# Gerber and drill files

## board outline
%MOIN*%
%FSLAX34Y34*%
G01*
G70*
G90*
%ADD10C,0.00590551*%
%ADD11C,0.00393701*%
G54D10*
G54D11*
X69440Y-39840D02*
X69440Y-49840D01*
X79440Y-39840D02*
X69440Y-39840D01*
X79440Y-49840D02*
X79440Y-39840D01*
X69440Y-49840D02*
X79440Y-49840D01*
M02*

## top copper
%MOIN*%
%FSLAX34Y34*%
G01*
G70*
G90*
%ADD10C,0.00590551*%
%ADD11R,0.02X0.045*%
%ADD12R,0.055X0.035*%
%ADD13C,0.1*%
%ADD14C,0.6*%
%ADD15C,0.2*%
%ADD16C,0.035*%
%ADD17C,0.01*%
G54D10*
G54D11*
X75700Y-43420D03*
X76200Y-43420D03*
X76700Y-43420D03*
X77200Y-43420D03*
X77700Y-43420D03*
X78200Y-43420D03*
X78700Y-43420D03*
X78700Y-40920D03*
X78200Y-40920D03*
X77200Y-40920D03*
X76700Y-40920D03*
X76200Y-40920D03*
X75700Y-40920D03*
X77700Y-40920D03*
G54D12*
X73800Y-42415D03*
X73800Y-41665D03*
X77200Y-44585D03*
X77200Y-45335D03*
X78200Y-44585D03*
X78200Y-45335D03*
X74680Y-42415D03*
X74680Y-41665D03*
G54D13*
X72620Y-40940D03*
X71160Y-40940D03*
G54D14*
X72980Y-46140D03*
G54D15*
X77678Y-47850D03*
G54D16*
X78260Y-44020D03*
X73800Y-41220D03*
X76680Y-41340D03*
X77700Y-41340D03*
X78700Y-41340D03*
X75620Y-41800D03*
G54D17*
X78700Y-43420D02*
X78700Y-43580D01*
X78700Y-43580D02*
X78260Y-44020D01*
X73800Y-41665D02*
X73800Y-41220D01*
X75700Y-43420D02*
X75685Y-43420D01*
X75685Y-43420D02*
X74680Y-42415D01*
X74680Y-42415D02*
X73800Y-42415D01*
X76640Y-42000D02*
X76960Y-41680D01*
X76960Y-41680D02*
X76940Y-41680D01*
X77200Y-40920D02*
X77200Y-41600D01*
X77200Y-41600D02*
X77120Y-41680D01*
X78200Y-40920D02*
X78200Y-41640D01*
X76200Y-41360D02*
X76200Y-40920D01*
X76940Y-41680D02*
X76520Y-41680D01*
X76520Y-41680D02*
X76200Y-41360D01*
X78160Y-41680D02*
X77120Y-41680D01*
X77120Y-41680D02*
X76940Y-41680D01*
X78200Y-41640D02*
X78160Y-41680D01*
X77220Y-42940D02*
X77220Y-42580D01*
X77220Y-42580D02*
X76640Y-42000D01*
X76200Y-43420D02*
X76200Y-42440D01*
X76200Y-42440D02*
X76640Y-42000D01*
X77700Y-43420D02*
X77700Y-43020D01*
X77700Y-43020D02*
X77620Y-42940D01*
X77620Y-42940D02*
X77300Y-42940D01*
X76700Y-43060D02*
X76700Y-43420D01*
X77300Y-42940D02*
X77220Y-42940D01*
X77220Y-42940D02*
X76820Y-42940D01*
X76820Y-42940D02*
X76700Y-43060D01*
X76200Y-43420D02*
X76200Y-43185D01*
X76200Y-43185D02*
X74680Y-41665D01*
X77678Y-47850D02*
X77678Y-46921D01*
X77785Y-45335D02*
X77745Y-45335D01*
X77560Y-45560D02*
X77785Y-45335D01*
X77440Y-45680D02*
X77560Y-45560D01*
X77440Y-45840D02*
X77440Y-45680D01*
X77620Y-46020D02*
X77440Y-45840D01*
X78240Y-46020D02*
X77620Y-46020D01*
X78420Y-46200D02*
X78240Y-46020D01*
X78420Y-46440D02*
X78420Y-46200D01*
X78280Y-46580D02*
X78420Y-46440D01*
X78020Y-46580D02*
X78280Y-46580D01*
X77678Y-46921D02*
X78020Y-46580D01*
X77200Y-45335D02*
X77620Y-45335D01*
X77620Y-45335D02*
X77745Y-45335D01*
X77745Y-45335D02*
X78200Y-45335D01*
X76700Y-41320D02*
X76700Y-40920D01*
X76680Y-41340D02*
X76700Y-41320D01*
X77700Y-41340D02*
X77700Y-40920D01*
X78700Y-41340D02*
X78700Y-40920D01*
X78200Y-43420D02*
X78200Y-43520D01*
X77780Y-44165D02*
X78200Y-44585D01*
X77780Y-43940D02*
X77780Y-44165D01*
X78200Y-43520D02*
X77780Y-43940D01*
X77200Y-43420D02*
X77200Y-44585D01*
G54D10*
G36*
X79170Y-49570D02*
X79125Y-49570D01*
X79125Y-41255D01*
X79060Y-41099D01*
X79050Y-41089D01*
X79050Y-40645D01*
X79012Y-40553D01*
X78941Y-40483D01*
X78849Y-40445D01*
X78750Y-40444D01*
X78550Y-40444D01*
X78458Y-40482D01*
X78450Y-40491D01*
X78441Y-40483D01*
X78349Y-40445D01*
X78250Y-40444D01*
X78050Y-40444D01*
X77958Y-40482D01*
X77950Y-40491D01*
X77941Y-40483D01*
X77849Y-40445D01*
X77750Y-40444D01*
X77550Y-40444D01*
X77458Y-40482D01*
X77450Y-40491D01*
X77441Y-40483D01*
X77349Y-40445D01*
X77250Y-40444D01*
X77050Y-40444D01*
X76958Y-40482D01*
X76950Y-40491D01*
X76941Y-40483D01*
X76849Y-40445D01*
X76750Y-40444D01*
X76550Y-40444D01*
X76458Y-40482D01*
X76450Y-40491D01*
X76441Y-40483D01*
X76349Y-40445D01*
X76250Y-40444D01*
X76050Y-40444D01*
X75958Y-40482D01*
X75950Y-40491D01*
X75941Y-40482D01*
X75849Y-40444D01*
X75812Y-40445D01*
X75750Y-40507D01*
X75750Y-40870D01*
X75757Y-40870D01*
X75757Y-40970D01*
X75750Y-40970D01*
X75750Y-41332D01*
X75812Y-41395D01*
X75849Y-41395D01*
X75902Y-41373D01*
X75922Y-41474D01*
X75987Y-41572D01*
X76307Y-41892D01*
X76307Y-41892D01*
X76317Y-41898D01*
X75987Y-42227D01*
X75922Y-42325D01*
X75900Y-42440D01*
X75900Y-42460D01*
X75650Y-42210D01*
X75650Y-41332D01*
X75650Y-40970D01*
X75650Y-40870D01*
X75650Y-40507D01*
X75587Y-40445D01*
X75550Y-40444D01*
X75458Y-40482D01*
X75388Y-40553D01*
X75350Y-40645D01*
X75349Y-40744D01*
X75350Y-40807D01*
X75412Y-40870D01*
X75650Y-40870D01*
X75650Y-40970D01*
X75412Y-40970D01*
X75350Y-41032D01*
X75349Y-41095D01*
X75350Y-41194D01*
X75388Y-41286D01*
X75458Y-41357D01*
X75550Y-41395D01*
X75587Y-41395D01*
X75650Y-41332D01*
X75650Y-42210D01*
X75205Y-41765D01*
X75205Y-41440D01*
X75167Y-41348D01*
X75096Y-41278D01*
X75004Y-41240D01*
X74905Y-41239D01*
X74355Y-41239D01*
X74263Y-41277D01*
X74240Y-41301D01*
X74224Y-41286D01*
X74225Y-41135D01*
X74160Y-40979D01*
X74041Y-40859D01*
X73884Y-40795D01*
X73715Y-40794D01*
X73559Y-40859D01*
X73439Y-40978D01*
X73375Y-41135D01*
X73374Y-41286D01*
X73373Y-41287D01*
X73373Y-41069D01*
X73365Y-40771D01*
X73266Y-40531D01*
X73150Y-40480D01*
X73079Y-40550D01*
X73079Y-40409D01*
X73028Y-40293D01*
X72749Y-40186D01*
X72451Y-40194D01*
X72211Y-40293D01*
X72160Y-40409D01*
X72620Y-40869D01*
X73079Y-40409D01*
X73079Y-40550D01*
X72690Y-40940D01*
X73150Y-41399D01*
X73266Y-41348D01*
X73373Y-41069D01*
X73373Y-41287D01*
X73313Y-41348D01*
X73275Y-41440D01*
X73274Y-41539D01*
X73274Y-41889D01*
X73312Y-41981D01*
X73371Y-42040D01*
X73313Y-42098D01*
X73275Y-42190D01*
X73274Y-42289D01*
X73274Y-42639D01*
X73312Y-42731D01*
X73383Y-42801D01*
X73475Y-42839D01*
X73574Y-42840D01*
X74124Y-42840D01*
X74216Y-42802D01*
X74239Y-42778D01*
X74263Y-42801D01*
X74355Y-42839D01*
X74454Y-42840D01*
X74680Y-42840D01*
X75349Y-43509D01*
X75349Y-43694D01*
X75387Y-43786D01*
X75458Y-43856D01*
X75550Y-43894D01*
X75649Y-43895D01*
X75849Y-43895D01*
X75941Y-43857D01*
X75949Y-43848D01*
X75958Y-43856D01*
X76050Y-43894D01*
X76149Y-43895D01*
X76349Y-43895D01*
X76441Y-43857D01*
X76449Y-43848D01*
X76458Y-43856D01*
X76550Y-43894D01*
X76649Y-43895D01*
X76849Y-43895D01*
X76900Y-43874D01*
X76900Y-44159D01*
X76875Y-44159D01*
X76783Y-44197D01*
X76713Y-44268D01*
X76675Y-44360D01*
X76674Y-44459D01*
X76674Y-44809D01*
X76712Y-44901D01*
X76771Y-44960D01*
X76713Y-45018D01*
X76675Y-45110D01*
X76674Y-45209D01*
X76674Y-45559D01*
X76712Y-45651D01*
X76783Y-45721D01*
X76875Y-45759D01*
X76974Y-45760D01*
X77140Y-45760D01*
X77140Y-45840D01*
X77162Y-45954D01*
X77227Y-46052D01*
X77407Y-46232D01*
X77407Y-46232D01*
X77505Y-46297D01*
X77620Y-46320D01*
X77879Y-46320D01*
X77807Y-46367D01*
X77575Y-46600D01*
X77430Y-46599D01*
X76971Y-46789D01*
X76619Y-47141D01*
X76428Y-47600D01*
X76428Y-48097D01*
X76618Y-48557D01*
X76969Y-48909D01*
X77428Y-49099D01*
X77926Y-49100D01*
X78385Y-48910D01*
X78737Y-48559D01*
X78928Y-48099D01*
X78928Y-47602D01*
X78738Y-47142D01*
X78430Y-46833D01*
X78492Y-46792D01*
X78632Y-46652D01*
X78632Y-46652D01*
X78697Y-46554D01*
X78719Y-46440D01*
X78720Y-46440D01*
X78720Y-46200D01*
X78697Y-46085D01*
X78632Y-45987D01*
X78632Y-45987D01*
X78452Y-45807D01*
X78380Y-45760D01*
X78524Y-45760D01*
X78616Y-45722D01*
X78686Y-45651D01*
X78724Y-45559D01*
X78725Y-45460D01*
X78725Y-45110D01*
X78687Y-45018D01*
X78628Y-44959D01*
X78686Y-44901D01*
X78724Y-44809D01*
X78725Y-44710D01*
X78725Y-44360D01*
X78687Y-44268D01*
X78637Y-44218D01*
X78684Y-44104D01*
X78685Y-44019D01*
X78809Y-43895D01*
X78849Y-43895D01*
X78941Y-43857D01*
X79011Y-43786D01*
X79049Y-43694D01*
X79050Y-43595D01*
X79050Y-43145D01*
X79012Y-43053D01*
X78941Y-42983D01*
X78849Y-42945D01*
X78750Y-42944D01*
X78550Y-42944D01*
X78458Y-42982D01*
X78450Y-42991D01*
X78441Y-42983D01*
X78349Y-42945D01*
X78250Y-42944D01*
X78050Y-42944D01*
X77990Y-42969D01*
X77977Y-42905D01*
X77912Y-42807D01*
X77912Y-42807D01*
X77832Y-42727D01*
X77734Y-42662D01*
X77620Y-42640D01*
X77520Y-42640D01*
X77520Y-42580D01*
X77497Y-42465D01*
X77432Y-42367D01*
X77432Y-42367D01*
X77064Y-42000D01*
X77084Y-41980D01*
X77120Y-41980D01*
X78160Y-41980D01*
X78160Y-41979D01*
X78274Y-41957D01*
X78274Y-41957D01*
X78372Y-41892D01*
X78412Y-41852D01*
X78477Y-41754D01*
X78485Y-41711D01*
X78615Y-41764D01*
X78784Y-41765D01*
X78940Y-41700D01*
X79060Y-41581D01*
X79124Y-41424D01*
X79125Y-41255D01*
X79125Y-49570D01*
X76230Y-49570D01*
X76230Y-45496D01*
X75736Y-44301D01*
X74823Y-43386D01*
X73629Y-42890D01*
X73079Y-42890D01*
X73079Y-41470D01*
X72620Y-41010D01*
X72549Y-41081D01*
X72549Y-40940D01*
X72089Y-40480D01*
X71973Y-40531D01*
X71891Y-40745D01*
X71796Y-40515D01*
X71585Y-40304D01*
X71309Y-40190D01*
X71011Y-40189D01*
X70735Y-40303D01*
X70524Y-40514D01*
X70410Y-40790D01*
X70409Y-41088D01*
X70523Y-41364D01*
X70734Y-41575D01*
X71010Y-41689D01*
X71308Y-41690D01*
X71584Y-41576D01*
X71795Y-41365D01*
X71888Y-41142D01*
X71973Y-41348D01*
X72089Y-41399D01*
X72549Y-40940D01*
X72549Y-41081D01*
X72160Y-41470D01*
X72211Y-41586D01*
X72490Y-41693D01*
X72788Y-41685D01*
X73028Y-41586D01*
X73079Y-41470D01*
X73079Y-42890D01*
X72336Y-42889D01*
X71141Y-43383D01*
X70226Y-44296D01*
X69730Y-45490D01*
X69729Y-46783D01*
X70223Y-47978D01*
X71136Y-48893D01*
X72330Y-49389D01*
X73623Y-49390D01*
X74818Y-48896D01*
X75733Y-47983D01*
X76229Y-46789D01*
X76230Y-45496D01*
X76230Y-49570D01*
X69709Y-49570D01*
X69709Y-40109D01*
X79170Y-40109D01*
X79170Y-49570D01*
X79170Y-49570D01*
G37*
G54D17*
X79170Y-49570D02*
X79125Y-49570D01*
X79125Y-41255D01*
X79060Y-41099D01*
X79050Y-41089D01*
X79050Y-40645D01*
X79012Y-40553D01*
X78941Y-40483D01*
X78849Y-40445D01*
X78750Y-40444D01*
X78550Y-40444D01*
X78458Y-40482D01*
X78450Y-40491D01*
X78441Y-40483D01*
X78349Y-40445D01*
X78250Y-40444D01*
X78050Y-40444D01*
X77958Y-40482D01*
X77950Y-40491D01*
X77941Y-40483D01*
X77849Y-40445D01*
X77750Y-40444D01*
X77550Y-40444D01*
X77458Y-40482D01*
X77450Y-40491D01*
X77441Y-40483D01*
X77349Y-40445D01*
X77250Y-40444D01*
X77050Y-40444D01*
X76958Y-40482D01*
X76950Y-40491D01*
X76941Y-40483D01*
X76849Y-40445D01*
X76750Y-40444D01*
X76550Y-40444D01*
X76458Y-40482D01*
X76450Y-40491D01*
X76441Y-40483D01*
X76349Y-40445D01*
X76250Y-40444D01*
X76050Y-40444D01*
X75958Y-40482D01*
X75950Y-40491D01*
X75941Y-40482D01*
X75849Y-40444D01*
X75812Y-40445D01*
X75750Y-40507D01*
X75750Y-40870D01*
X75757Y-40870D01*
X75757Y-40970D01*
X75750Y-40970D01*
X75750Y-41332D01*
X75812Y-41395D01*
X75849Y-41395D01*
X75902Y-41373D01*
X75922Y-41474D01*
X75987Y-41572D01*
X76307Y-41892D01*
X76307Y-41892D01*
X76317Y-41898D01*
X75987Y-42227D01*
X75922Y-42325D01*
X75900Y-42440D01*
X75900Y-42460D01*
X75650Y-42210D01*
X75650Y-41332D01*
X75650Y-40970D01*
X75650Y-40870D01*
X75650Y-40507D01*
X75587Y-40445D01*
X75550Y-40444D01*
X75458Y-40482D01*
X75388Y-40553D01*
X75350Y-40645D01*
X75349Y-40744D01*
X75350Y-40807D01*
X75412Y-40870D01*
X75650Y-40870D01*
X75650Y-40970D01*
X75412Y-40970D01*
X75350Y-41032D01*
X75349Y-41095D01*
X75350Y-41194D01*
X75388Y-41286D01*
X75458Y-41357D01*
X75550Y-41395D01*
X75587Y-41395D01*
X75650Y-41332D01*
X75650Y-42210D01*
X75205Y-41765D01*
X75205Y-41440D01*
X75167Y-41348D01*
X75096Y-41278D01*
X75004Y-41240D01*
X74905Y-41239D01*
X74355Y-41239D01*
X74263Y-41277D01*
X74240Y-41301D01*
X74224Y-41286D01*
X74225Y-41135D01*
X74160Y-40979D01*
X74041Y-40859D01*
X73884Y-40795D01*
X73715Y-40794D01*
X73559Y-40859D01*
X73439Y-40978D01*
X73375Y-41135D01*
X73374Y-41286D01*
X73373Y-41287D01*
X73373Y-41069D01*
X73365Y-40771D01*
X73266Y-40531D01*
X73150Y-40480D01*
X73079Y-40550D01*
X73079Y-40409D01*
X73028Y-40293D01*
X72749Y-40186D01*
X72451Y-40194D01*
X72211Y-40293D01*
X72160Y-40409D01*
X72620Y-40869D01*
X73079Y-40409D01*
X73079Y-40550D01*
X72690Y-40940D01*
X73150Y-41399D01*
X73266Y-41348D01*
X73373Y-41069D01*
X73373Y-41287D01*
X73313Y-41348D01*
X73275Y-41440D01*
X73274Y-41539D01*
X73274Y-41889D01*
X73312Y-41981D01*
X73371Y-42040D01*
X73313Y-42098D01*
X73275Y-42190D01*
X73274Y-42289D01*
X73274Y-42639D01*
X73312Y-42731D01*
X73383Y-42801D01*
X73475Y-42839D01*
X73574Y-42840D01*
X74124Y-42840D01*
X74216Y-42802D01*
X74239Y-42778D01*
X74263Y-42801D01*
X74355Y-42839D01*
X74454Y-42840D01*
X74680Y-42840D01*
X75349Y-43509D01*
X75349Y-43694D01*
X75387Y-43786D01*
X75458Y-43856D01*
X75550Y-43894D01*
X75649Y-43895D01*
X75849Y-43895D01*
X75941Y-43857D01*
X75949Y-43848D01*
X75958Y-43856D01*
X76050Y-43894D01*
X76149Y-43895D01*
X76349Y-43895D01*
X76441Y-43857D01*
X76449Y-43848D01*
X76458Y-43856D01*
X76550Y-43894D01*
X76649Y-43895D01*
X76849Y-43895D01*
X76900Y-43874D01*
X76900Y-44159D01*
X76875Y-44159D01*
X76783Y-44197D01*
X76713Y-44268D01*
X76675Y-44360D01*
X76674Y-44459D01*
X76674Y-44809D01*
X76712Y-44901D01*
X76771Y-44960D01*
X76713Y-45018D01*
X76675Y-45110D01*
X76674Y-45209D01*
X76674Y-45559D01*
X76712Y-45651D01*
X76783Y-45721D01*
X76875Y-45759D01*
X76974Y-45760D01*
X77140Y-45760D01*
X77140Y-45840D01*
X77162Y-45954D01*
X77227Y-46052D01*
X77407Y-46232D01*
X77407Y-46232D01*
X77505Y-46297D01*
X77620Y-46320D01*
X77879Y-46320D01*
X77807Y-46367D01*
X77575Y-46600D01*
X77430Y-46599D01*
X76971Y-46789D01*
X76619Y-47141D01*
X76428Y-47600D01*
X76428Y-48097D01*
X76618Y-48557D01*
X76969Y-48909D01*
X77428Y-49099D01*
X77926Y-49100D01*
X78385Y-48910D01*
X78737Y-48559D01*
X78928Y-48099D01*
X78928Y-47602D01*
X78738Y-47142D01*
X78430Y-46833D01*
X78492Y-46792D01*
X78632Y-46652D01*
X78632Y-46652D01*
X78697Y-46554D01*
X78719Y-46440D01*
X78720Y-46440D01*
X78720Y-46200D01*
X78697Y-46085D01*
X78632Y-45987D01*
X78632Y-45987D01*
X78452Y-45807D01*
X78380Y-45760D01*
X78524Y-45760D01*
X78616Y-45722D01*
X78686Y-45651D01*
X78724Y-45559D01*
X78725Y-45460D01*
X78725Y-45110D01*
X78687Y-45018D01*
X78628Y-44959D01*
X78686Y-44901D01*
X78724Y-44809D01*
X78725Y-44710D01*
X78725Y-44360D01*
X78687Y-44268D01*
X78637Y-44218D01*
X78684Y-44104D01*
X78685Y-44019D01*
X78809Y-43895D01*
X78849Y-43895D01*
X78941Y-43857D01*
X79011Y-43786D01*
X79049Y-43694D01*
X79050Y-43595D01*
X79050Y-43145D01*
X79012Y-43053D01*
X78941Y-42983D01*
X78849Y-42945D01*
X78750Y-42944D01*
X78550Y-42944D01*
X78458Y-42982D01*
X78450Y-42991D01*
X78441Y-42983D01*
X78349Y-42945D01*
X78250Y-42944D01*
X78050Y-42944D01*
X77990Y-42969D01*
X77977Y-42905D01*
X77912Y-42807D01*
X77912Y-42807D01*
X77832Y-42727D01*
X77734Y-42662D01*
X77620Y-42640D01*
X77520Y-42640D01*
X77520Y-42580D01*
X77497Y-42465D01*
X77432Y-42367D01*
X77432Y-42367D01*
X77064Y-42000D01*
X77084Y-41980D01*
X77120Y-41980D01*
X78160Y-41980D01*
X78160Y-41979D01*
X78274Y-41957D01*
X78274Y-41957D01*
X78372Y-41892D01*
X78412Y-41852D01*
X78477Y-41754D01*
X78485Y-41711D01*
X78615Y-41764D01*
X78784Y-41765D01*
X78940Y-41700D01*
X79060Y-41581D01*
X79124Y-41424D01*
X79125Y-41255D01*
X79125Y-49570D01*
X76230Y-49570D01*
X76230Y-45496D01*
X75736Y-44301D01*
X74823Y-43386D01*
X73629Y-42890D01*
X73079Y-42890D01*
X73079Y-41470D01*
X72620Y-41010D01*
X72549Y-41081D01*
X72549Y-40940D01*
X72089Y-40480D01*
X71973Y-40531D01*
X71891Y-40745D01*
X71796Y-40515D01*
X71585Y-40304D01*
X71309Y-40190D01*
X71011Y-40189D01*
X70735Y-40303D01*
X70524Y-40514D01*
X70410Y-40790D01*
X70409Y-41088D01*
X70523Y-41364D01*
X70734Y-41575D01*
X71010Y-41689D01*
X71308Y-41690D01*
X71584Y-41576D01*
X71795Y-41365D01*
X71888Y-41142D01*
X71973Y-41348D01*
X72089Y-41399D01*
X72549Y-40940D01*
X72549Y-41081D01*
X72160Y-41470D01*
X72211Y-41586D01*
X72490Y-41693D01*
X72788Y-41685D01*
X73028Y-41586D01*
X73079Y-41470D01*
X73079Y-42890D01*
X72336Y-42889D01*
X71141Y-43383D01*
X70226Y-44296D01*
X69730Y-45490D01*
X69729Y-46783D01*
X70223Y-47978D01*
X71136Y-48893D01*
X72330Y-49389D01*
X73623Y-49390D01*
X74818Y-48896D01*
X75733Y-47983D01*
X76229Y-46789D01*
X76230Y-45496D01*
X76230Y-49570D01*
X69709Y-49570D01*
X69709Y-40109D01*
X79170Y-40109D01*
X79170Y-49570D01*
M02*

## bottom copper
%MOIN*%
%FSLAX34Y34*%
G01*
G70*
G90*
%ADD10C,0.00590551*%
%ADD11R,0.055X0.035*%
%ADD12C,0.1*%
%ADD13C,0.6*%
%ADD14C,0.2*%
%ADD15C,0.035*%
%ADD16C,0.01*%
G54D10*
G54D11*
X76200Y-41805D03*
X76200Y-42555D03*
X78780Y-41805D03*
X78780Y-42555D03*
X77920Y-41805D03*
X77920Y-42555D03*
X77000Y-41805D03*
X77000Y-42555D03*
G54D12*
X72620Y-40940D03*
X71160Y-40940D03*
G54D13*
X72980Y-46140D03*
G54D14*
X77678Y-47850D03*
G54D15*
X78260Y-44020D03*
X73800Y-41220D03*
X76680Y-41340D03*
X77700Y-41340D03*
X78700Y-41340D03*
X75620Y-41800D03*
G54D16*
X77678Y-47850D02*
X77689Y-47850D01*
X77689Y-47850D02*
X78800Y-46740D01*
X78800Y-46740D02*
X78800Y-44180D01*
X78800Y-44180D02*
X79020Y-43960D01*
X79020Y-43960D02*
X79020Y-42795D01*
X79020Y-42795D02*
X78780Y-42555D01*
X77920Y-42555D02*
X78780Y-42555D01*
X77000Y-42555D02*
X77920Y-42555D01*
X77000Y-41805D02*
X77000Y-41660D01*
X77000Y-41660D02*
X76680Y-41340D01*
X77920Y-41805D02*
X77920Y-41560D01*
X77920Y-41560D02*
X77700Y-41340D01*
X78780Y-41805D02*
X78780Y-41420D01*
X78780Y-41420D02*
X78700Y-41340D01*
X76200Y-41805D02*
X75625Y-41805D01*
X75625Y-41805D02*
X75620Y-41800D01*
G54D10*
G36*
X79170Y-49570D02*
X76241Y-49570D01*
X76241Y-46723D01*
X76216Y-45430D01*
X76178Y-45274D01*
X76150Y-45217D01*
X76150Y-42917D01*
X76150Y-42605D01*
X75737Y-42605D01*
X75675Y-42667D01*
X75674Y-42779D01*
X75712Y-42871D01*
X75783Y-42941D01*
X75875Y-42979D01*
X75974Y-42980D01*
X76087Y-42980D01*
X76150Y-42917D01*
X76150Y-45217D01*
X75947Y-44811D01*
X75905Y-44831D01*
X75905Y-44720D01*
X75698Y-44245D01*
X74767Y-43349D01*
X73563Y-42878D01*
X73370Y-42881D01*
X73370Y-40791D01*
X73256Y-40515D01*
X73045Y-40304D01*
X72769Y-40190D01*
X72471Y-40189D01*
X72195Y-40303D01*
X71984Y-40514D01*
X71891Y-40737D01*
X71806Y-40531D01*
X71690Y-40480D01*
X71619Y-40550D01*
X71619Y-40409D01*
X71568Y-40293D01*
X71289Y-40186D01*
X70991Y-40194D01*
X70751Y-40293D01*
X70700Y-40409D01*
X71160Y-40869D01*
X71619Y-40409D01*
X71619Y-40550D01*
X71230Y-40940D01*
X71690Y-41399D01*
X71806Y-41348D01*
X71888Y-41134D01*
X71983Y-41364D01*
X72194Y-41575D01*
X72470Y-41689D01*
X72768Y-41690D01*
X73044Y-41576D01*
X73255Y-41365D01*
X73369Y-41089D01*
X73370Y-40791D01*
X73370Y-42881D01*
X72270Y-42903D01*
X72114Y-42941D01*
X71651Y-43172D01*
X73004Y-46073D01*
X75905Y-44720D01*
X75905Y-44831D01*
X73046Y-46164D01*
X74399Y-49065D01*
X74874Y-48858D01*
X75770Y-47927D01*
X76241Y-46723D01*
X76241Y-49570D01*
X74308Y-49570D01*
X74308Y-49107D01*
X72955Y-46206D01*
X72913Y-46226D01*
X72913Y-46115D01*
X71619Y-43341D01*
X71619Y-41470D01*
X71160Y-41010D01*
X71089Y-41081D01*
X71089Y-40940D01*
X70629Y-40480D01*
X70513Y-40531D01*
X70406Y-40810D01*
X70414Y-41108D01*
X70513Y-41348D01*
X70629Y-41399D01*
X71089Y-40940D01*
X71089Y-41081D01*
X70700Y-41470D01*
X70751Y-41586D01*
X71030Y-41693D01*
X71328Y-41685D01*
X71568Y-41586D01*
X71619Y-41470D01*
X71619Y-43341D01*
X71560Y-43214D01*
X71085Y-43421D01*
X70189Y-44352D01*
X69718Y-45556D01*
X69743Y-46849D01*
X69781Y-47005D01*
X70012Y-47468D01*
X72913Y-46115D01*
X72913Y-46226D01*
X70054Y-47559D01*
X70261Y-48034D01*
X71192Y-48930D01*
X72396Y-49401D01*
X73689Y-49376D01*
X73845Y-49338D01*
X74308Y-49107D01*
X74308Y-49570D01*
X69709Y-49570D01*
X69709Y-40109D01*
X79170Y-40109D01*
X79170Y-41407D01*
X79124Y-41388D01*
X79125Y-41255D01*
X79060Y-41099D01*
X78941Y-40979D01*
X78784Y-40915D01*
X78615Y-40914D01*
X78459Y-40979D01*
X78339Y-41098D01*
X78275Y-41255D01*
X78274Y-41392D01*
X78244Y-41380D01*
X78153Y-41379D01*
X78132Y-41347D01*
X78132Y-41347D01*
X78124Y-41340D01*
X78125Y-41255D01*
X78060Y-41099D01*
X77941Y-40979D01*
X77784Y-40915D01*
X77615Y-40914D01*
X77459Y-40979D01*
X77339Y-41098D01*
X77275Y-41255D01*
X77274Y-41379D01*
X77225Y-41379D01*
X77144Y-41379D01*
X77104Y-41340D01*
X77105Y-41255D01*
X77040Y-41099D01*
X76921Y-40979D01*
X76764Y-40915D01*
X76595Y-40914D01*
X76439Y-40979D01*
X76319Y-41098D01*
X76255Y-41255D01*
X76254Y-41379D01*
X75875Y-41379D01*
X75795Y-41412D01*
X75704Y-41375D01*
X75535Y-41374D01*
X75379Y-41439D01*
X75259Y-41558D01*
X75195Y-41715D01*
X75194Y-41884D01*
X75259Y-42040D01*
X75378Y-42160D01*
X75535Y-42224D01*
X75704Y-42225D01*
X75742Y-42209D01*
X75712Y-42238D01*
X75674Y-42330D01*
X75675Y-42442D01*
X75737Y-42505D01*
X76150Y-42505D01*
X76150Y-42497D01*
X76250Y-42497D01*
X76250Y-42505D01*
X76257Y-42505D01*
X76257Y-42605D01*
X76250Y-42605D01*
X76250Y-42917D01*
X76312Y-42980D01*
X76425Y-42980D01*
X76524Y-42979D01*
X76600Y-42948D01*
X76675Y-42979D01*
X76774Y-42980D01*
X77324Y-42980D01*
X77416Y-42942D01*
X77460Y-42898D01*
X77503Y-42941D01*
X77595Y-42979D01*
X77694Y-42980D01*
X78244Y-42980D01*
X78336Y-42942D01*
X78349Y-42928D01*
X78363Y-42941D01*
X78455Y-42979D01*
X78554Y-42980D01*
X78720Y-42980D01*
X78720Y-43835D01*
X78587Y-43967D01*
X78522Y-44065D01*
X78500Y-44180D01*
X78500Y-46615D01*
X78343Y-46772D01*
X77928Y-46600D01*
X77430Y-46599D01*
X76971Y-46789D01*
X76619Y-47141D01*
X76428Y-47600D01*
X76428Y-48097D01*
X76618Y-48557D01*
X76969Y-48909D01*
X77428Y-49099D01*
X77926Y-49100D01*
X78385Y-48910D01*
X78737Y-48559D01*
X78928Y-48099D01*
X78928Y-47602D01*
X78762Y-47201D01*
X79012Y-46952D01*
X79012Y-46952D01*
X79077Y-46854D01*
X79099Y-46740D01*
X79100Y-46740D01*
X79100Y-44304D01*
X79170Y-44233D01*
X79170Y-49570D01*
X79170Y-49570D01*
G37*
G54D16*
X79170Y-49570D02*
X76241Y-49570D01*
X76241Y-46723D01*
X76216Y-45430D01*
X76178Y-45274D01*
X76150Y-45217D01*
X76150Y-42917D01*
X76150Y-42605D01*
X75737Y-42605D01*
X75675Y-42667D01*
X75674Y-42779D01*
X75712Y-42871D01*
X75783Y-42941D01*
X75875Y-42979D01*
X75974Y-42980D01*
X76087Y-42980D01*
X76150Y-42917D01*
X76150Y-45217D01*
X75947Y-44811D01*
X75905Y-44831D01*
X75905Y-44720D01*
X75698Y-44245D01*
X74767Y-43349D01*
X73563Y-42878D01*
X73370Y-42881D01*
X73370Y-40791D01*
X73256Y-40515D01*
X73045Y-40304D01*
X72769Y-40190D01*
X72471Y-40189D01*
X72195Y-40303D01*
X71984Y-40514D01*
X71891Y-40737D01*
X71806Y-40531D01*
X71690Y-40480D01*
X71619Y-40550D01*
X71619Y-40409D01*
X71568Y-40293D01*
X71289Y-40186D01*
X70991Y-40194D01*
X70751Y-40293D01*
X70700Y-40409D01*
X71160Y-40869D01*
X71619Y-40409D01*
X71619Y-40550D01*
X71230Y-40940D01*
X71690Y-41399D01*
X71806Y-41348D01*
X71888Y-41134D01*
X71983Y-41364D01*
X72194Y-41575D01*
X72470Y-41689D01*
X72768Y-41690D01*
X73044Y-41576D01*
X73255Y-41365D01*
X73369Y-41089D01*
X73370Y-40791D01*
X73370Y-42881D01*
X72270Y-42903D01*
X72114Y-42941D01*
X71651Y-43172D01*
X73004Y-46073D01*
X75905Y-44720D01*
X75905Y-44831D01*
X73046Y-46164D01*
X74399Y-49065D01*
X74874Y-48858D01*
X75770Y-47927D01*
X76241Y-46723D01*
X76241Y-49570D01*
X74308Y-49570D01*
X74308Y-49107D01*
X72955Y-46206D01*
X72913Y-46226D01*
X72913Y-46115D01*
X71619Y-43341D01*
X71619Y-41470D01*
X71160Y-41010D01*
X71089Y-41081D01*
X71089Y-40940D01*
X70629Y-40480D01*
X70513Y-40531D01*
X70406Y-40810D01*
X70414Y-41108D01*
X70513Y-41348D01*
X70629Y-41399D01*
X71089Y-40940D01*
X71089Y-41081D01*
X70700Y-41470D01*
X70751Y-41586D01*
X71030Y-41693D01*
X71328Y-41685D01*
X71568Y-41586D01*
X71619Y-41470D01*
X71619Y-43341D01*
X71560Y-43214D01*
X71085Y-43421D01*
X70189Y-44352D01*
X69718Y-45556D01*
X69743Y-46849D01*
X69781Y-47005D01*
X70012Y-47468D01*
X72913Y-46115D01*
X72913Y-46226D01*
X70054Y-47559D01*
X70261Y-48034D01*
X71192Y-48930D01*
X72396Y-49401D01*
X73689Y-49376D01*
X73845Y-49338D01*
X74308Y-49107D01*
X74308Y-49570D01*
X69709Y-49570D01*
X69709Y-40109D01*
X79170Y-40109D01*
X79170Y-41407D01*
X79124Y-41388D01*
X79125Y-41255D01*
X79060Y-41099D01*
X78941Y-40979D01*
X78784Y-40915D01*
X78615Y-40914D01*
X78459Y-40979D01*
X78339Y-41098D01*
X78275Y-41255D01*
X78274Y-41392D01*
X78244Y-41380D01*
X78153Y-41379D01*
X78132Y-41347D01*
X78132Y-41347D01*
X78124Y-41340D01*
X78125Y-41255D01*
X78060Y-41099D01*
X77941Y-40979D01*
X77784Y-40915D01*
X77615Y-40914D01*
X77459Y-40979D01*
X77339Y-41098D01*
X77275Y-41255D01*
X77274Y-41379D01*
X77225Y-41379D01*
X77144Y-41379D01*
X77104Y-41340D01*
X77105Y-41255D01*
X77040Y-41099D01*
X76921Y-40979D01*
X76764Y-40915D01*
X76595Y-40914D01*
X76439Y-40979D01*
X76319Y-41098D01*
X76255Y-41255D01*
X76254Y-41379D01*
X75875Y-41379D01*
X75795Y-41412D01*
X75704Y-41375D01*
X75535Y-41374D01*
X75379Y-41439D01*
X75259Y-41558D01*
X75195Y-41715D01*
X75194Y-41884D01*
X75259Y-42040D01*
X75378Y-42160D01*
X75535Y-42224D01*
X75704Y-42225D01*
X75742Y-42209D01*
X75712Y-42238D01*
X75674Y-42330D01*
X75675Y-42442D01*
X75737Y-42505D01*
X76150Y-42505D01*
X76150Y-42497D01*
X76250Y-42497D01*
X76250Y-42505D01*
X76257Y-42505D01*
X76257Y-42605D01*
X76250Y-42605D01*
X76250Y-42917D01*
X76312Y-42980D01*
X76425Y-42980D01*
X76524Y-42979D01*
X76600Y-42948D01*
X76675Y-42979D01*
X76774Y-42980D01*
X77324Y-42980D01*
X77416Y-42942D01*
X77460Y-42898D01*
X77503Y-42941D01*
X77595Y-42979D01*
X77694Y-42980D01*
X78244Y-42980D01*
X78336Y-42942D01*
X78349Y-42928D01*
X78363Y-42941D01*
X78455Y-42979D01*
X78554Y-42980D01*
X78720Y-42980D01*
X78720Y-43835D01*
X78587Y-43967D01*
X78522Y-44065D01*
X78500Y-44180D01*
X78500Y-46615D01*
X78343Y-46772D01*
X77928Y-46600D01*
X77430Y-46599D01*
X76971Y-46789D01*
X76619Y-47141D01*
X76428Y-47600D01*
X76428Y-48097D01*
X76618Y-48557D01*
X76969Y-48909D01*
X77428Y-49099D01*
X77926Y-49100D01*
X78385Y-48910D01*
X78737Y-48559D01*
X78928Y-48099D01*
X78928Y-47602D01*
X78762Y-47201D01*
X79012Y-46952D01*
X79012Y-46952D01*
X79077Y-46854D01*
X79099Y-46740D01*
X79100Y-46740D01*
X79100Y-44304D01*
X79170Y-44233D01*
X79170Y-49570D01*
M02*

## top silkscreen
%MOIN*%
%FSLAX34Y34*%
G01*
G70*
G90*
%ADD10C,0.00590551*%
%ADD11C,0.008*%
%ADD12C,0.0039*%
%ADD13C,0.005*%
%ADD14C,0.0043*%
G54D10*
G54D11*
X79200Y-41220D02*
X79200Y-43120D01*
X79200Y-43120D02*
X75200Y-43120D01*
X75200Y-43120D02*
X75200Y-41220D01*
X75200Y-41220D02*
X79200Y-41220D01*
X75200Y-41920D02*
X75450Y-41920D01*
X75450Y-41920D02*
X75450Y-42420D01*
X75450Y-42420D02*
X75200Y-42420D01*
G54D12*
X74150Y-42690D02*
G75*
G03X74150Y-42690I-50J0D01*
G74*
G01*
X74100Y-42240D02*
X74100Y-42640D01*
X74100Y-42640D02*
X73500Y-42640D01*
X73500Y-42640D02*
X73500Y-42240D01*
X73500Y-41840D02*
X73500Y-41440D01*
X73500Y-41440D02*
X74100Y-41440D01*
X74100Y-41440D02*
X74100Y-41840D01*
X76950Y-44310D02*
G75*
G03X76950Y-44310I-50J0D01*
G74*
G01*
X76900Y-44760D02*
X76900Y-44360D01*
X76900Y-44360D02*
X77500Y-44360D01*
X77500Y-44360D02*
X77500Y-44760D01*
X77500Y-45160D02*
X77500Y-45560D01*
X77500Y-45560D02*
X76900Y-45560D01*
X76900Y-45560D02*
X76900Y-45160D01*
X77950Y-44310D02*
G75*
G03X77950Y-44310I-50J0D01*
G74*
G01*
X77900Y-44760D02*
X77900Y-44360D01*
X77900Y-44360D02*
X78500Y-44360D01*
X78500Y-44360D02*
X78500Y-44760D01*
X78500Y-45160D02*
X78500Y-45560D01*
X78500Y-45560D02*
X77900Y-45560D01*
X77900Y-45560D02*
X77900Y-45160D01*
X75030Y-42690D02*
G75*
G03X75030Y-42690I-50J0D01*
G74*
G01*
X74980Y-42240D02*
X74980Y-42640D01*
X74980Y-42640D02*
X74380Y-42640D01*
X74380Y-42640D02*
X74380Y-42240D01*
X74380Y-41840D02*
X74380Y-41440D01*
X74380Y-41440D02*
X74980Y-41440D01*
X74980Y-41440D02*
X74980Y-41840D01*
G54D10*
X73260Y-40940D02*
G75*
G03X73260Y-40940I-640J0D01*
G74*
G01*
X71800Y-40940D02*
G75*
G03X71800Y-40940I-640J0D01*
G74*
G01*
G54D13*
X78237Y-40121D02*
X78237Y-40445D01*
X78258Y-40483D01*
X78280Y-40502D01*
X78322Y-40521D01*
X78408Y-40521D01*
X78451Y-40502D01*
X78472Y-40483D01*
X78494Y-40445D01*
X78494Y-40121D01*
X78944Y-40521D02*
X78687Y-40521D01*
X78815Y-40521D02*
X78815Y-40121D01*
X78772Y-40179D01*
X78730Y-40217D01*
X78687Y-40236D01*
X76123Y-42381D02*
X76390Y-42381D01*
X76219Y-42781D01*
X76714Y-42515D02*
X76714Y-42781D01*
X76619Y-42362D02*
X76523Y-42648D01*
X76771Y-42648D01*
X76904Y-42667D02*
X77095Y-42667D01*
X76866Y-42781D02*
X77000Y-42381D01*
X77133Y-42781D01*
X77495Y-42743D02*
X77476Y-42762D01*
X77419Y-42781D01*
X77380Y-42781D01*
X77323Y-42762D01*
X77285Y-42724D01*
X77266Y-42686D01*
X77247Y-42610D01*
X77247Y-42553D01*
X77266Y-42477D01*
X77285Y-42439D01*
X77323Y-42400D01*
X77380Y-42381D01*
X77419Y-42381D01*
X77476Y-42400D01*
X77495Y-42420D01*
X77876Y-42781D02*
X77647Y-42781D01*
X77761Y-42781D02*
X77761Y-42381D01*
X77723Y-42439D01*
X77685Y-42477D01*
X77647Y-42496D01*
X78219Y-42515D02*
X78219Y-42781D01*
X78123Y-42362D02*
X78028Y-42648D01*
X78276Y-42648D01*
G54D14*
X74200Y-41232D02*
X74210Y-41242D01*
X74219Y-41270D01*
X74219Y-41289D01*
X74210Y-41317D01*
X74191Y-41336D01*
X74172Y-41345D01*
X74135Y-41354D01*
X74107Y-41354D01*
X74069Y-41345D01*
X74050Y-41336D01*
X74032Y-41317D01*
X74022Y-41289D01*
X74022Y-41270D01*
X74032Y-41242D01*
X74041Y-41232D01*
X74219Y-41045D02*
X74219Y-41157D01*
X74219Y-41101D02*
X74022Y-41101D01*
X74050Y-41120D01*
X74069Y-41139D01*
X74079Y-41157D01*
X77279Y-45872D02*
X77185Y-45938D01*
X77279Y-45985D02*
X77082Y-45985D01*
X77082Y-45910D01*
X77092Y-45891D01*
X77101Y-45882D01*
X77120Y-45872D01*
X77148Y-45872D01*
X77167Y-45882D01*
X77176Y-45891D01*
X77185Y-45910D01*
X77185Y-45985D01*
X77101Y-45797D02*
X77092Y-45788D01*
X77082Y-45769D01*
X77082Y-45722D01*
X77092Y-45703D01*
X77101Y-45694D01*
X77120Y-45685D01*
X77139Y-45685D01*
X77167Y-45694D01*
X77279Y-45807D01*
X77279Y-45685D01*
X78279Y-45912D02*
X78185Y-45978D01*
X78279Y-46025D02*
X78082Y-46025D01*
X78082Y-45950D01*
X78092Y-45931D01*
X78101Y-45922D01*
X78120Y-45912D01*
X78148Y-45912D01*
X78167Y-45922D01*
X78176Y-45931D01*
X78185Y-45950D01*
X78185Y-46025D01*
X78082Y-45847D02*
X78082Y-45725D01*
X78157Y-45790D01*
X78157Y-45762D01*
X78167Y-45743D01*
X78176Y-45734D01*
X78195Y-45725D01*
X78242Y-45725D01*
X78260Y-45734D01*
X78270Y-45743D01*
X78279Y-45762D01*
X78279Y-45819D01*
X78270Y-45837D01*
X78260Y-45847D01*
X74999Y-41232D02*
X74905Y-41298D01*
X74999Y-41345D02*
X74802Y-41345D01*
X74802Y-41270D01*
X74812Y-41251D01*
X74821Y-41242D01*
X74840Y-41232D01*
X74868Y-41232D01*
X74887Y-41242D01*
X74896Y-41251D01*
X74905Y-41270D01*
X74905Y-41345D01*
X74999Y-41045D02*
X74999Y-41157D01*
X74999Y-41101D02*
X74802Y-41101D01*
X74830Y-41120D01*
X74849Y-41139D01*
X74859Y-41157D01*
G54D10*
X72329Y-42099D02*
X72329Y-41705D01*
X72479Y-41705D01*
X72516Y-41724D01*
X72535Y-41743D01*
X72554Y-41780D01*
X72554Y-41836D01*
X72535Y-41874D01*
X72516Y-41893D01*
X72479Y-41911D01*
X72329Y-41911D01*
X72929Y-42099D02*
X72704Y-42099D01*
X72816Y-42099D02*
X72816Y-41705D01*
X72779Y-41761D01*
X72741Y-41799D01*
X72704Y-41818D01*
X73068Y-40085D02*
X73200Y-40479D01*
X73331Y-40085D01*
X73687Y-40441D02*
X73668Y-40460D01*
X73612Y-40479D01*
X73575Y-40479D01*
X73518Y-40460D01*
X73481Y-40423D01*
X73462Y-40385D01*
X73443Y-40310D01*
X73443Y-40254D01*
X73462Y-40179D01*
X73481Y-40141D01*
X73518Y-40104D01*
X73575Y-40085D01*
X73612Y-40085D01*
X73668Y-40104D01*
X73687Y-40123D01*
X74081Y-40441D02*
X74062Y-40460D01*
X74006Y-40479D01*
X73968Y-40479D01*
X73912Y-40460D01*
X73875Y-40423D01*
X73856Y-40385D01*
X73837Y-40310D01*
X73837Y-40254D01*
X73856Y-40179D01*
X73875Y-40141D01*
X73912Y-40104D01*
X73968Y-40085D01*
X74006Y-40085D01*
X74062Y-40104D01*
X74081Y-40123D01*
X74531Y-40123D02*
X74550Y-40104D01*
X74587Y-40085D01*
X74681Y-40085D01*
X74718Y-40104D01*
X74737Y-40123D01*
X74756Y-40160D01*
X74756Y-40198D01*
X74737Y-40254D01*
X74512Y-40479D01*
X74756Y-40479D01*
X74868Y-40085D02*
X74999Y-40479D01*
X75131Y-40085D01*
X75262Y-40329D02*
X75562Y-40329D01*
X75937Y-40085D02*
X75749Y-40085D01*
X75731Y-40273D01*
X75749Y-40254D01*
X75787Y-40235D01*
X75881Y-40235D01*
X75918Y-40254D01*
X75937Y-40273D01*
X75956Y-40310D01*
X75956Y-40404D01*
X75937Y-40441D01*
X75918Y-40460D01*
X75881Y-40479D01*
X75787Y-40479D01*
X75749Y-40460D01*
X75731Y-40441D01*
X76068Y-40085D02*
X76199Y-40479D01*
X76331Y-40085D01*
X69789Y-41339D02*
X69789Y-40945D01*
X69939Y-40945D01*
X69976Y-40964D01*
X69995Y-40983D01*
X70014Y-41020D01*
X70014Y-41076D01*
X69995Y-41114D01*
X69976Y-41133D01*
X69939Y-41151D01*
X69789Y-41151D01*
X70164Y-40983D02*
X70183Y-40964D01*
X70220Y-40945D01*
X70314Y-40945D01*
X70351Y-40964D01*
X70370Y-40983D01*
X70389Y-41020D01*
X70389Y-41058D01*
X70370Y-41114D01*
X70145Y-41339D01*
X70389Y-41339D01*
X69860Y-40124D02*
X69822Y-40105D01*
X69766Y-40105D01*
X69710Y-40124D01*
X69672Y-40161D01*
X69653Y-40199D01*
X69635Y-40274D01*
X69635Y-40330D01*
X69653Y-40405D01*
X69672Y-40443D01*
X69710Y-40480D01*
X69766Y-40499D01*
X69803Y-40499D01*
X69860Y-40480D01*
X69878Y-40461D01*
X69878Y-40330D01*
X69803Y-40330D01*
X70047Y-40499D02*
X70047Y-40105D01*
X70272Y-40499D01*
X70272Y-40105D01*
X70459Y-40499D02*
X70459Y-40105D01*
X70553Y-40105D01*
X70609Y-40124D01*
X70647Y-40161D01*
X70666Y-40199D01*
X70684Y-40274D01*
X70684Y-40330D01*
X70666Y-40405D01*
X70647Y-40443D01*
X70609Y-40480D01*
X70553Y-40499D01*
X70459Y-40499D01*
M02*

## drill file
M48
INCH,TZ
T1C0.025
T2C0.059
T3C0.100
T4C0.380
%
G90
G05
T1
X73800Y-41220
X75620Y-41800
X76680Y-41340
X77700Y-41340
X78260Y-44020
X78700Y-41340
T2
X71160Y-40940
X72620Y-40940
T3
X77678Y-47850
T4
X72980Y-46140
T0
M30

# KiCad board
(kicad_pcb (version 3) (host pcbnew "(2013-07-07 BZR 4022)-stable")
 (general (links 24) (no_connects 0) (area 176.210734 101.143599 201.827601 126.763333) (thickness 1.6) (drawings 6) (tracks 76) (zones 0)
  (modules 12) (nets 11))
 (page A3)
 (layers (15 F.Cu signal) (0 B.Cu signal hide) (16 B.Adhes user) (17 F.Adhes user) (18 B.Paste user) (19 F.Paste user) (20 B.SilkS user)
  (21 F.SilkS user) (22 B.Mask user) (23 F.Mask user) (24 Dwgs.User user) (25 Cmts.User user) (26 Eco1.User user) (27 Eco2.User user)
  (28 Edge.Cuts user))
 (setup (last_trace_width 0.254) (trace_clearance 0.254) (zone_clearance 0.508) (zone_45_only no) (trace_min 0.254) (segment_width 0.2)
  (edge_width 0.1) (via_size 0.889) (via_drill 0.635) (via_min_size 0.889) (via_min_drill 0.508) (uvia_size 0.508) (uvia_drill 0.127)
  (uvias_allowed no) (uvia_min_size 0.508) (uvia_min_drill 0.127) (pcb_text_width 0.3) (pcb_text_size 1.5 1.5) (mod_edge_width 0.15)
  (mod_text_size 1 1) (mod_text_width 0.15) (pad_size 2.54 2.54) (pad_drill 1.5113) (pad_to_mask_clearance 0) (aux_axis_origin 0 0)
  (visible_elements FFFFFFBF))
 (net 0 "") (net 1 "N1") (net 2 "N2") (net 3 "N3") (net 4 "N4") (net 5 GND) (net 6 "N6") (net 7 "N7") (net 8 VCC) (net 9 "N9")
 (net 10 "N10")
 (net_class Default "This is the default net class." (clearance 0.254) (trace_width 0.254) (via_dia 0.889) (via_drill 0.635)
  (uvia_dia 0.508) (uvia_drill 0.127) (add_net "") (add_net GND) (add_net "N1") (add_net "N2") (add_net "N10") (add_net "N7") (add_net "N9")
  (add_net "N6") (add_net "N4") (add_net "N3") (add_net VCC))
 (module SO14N (layer F.Cu) (at 196.088 106.9848)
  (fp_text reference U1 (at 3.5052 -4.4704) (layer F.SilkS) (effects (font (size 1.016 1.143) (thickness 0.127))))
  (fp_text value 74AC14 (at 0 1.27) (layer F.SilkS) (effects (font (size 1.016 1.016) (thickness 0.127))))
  (fp_line (start 5.08 -2.286) (end 5.08 2.54) (layer F.SilkS) (width 0.2032))
  (fp_line (start 5.08 2.54) (end -5.08 2.54) (layer F.SilkS) (width 0.2032))
  (fp_line (start -5.08 2.54) (end -5.08 -2.286) (layer F.SilkS) (width 0.2032))
  (fp_line (start -5.08 -2.286) (end 5.08 -2.286) (layer F.SilkS) (width 0.2032))
  (fp_line (start -5.08 -0.508) (end -4.445 -0.508) (layer F.SilkS) (width 0.2032))
  (fp_line (start -4.445 -0.508) (end -4.445 0.762) (layer F.SilkS) (width 0.2032))
  (fp_line (start -4.445 0.762) (end -5.08 0.762) (layer F.SilkS) (width 0.2032))
  (pad 1 smd rect (at -3.81 3.302) (size 0.508 1.143) (layers F.Cu F.Paste F.Mask) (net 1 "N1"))
  (pad 2 smd rect (at -2.54 3.302) (size 0.508 1.143) (layers F.Cu F.Paste F.Mask) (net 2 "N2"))
  (pad 3 smd rect (at -1.27 3.302) (size 0.508 1.143) (layers F.Cu F.Paste F.Mask) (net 2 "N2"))
  (pad 4 smd rect (at 0 3.302) (size 0.508 1.143) (layers F.Cu F.Paste F.Mask) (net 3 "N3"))
  (pad 5 smd rect (at 1.27 3.302) (size 0.508 1.143) (layers F.Cu F.Paste F.Mask) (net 2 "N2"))
  (pad 6 smd rect (at 2.54 3.302) (size 0.508 1.143) (layers F.Cu F.Paste F.Mask) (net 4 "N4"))
  (pad 7 smd rect (at 3.81 3.302) (size 0.508 1.143) (layers F.Cu F.Paste F.Mask) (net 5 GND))
  (pad 8 smd rect (at 3.81 -3.048) (size 0.508 1.143) (layers F.Cu F.Paste F.Mask) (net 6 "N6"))
  (pad 9 smd rect (at 2.54 -3.048) (size 0.508 1.143) (layers F.Cu F.Paste F.Mask) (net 2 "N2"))
  (pad 11 smd rect (at 0 -3.048) (size 0.508 1.143) (layers F.Cu F.Paste F.Mask) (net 2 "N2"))
  (pad 12 smd rect (at -1.27 -3.048) (size 0.508 1.143) (layers F.Cu F.Paste F.Mask) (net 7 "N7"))
  (pad 13 smd rect (at -2.54 -3.048) (size 0.508 1.143) (layers F.Cu F.Paste F.Mask) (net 2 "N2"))
  (pad 14 smd rect (at -3.81 -3.048) (size 0.508 1.143) (layers F.Cu F.Paste F.Mask) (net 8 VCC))
  (pad 10 smd rect (at 1.27 -3.048) (size 0.508 1.143) (layers F.Cu F.Paste F.Mask) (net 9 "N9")))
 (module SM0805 (layer F.Cu) (at 187.452 106.7816 90)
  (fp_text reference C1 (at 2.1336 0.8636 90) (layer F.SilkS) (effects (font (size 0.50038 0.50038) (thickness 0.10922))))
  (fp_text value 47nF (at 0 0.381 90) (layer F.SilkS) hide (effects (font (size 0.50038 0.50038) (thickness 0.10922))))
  (fp_circle (center -1.651 0.762) (end -1.651 0.635) (layer F.SilkS) (width 0.09906))
  (fp_line (start -0.508 0.762) (end -1.524 0.762) (layer F.SilkS) (width 0.09906))
  (fp_line (start -1.524 0.762) (end -1.524 -0.762) (layer F.SilkS) (width 0.09906))
  (fp_line (start -1.524 -0.762) (end -0.508 -0.762) (layer F.SilkS) (width 0.09906))
  (fp_line (start 0.508 -0.762) (end 1.524 -0.762) (layer F.SilkS) (width 0.09906))
  (fp_line (start 1.524 -0.762) (end 1.524 0.762) (layer F.SilkS) (width 0.09906))
  (fp_line (start 1.524 0.762) (end 0.508 0.762) (layer F.SilkS) (width 0.09906))
  (pad 1 smd rect (at -0.9525 0 90) (size 0.889 1.397) (layers F.Cu F.Paste F.Mask) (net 1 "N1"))
  (pad 2 smd rect (at 0.9525 0 90) (size 0.889 1.397) (layers F.Cu F.Paste F.Mask) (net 5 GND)))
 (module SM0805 (layer B.Cu) (at 193.548 107.1372 270)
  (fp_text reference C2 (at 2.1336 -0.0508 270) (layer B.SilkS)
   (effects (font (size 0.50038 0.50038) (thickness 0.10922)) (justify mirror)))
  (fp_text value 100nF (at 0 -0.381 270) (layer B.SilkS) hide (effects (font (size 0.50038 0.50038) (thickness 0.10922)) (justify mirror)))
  (pad 1 smd rect (at -0.9525 0 270) (size 0.889 1.397) (layers B.Cu B.Paste B.Mask) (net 8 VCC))
  (pad 2 smd rect (at 0.9525 0 270) (size 0.889 1.397) (layers B.Cu B.Paste B.Mask) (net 5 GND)))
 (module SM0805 (layer F.Cu) (at 196.088 114.1984 270)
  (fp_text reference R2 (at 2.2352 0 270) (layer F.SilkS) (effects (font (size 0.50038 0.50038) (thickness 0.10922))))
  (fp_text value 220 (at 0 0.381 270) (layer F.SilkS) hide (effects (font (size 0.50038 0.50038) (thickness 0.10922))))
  (fp_circle (center -1.651 0.762) (end -1.651 0.635) (layer F.SilkS) (width 0.09906))
  (fp_line (start -0.508 0.762) (end -1.524 0.762) (layer F.SilkS) (width 0.09906))
  (fp_line (start -1.524 0.762) (end -1.524 -0.762) (layer F.SilkS) (width 0.09906))
  (fp_line (start -1.524 -0.762) (end -0.508 -0.762) (layer F.SilkS) (width 0.09906))
  (fp_line (start 0.508 -0.762) (end 1.524 -0.762) (layer F.SilkS) (width 0.09906))
  (fp_line (start 1.524 -0.762) (end 1.524 0.762) (layer F.SilkS) (width 0.09906))
  (fp_line (start 1.524 0.762) (end 0.508 0.762) (layer F.SilkS) (width 0.09906))
  (pad 1 smd rect (at -0.9525 0 270) (size 0.889 1.397) (layers F.Cu F.Paste F.Mask) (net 3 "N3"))
  (pad 2 smd rect (at 0.9525 0 270) (size 0.889 1.397) (layers F.Cu F.Paste F.Mask) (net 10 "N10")))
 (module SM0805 (layer F.Cu) (at 198.628 114.1984 270)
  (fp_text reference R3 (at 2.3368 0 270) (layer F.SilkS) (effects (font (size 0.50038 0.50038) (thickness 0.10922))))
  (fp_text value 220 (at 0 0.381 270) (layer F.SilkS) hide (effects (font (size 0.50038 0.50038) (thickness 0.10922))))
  (fp_circle (center -1.651 0.762) (end -1.651 0.635) (layer F.SilkS) (width 0.09906))
  (fp_line (start -0.508 0.762) (end -1.524 0.762) (layer F.SilkS) (width 0.09906))
  (fp_line (start -1.524 0.762) (end -1.524 -0.762) (layer F.SilkS) (width 0.09906))
  (fp_line (start -1.524 -0.762) (end -0.508 -0.762) (layer F.SilkS) (width 0.09906))
  (fp_line (start 0.508 -0.762) (end 1.524 -0.762) (layer F.SilkS) (width 0.09906))
  (fp_line (start 1.524 -0.762) (end 1.524 0.762) (layer F.SilkS) (width 0.09906))
  (fp_line (start 1.524 0.762) (end 0.508 0.762) (layer F.SilkS) (width 0.09906))
  (pad 1 smd rect (at -0.9525 0 270) (size 0.889 1.397) (layers F.Cu F.Paste F.Mask) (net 4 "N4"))
  (pad 2 smd rect (at 0.9525 0 270) (size 0.889 1.397) (layers F.Cu F.Paste F.Mask) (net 10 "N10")))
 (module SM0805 (layer B.Cu) (at 200.1012 107.1372 270)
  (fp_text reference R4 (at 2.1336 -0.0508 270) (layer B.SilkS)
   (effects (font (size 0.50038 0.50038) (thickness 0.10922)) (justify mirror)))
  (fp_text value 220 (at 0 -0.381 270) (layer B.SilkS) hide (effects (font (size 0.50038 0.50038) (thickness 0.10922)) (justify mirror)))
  (pad 1 smd rect (at -0.9525 0 270) (size 0.889 1.397) (layers B.Cu B.Paste B.Mask) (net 6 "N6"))
  (pad 2 smd rect (at 0.9525 0 270) (size 0.889 1.397) (layers B.Cu B.Paste B.Mask) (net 10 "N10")))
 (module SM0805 (layer B.Cu) (at 197.9168 107.1372 270)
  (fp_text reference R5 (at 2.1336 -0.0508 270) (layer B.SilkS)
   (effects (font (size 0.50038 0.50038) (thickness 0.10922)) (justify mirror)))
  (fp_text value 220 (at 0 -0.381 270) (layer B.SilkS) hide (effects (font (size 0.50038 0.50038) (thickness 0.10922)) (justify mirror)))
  (pad 1 smd rect (at -0.9525 0 270) (size 0.889 1.397) (layers B.Cu B.Paste B.Mask) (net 9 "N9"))
  (pad 2 smd rect (at 0.9525 0 270) (size 0.889 1.397) (layers B.Cu B.Paste B.Mask) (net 10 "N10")))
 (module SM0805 (layer B.Cu) (at 195.58 107.1372 270)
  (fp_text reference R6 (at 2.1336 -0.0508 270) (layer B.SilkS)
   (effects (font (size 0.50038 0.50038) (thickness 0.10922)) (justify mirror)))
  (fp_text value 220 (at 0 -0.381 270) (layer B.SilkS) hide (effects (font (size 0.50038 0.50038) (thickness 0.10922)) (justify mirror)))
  (pad 1 smd rect (at -0.9525 0 270) (size 0.889 1.397) (layers B.Cu B.Paste B.Mask) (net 7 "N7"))
  (pad 2 smd rect (at 0.9525 0 270) (size 0.889 1.397) (layers B.Cu B.Paste B.Mask) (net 10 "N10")))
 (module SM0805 (layer F.Cu) (at 189.6872 106.7816 90)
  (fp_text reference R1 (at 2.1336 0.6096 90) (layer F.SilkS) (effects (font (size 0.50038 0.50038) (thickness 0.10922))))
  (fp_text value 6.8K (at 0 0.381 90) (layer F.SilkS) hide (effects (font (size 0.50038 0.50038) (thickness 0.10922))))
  (fp_circle (center -1.651 0.762) (end -1.651 0.635) (layer F.SilkS) (width 0.09906))
  (fp_line (start -0.508 0.762) (end -1.524 0.762) (layer F.SilkS) (width 0.09906))
  (fp_line (start -1.524 0.762) (end -1.524 -0.762) (layer F.SilkS) (width 0.09906))
  (fp_line (start -1.524 -0.762) (end -0.508 -0.762) (layer F.SilkS) (width 0.09906))
  (fp_line (start 0.508 -0.762) (end 1.524 -0.762) (layer F.SilkS) (width 0.09906))
  (fp_line (start 1.524 -0.762) (end 1.524 0.762) (layer F.SilkS) (width 0.09906))
  (fp_line (start 1.524 0.762) (end 0.508 0.762) (layer F.SilkS) (width 0.09906))
  (pad 1 smd rect (at -0.9525 0 90) (size 0.889 1.397) (layers F.Cu F.Paste F.Mask) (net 1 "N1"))
  (pad 2 smd rect (at 0.9525 0 90) (size 0.889 1.397) (layers F.Cu F.Paste F.Mask) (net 2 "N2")))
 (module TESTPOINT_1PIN (layer F.Cu) (at 184.4548 103.9876)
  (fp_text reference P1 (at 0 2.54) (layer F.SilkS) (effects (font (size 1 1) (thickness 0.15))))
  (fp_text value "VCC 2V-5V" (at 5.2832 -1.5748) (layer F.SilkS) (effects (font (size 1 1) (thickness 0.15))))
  (fp_circle (center 0 0) (end 1.6256 0) (layer F.SilkS) (width 0.15))
  (pad 1 thru_hole circle (at 0 0) (size 2.54 2.54) (drill 1.5113) (layers *.Cu *.Mask F.SilkS) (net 8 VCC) (solder_mask_margin 0.254)))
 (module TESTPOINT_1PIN (layer F.Cu) (at 180.7464 103.9876)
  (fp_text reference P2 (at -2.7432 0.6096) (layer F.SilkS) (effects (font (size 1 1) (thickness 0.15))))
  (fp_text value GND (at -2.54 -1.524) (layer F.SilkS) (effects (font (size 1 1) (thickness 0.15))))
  (fp_circle (center 0 0) (end 1.6256 0) (layer F.SilkS) (width 0.15))
  (pad 1 thru_hole circle (at 0 0) (size 2.54 2.54) (drill 1.5113) (layers *.Cu *.Mask F.SilkS) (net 5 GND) (solder_mask_margin 0.254)))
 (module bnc (layer B.Cu) (at 185.3692 117.1956 340)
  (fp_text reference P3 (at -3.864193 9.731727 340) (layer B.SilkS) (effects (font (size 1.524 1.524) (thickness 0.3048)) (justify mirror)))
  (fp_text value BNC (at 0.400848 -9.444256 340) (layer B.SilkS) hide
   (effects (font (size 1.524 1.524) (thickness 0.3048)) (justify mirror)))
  (pad 2 thru_hole circle (at 0 0 340) (size 15.24 15.24) (drill 9.652) (layers *.Cu *.Mask B.SilkS) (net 5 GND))
  (pad 1 thru_hole circle (at 12.7 0 340) (size 5.08 5.08) (drill 2.54) (layers *.Cu *.Mask B.SilkS) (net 10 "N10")))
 (gr_line (start 176.3776 101.1936) (end 176.3776 126.5936) (angle 90) (layer Edge.Cuts) (width 0.1))
 (gr_line (start 201.7776 101.1936) (end 176.3776 101.1936) (angle 90) (layer Edge.Cuts) (width 0.1))
 (gr_line (start 201.7776 126.5936) (end 201.7776 101.1936) (angle 90) (layer Edge.Cuts) (width 0.1))
 (gr_line (start 176.3776 126.5936) (end 201.7776 126.5936) (angle 90) (layer Edge.Cuts) (width 0.1))
 (segment (start 199.898 110.2868) (end 199.898 110.6932) (width 0.254) (layer F.Cu) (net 5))
 (via (at 198.7804 111.8108) (size 0.889) (layers F.Cu B.Cu) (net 5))
 (segment (start 199.898 110.6932) (end 198.7804 111.8108) (width 0.254) (layer F.Cu) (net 5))
 (segment (start 187.452 105.8291) (end 187.452 104.6988) (width 0.254) (layer F.Cu) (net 5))
 (via (at 187.452 104.6988) (size 0.889) (layers F.Cu B.Cu) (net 5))
 (segment (start 192.278 110.2868) (end 192.2399 110.2868) (width 0.254) (layer F.Cu) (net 1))
 (segment (start 192.2399 110.2868) (end 189.6872 107.7341) (width 0.254) (layer F.Cu) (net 1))
 (segment (start 189.6872 107.7341) (end 187.452 107.7341) (width 0.254) (layer F.Cu) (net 1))
 (segment (start 194.6656 106.68) (end 195.4784 105.8672) (width 0.254) (layer F.Cu) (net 2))
 (segment (start 195.4784 105.8672) (end 195.4276 105.8672) (width 0.254) (layer F.Cu) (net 2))
 (segment (start 196.088 103.9368) (end 196.088 105.664) (width 0.254) (layer F.Cu) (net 2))
 (segment (start 196.088 105.664) (end 195.8848 105.8672) (width 0.254) (layer F.Cu) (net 2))
 (segment (start 198.628 103.9368) (end 198.628 105.7656) (width 0.254) (layer F.Cu) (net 2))
 (segment (start 193.548 105.0544) (end 193.548 103.9368) (width 0.254) (layer F.Cu) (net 2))
 (segment (start 195.4276 105.8672) (end 194.3608 105.8672) (width 0.254) (layer F.Cu) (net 2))
 (segment (start 194.3608 105.8672) (end 193.548 105.0544) (width 0.254) (layer F.Cu) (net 2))
 (segment (start 198.5264 105.8672) (end 195.8848 105.8672) (width 0.254) (layer F.Cu) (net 2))
 (segment (start 195.8848 105.8672) (end 195.4276 105.8672) (width 0.254) (layer F.Cu) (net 2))
 (segment (start 198.628 105.7656) (end 198.5264 105.8672) (width 0.254) (layer F.Cu) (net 2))
 (segment (start 196.1388 109.0676) (end 196.1388 108.1532) (width 0.254) (layer F.Cu) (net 2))
 (segment (start 196.1388 108.1532) (end 194.6656 106.68) (width 0.254) (layer F.Cu) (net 2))
 (segment (start 193.548 110.2868) (end 193.548 107.7976) (width 0.254) (layer F.Cu) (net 2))
 (segment (start 193.548 107.7976) (end 194.6656 106.68) (width 0.254) (layer F.Cu) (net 2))
 (segment (start 197.358 110.2868) (end 197.358 109.2708) (width 0.254) (layer F.Cu) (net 2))
 (segment (start 197.358 109.2708) (end 197.1548 109.0676) (width 0.254) (layer F.Cu) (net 2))
 (segment (start 197.1548 109.0676) (end 196.342 109.0676) (width 0.254) (layer F.Cu) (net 2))
 (segment (start 194.818 109.3724) (end 194.818 110.2868) (width 0.254) (layer F.Cu) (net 2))
 (segment (start 196.342 109.0676) (end 196.1388 109.0676) (width 0.254) (layer F.Cu) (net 2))
 (segment (start 196.1388 109.0676) (end 195.1228 109.0676) (width 0.254) (layer F.Cu) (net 2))
 (segment (start 195.1228 109.0676) (end 194.818 109.3724) (width 0.254) (layer F.Cu) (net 2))
 (segment (start 193.548 110.2868) (end 193.548 109.6899) (width 0.254) (layer F.Cu) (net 2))
 (segment (start 193.548 109.6899) (end 189.6872 105.8291) (width 0.254) (layer F.Cu) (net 2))
 (segment (start 197.303296 121.539256) (end 197.303296 119.180704) (width 0.254) (layer F.Cu) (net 10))
 (segment (start 197.5739 115.1509) (end 197.4723 115.1509) (width 0.254) (layer F.Cu) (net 10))
 (segment (start 197.0024 115.7224) (end 197.5739 115.1509) (width 0.254) (layer F.Cu) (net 10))
 (segment (start 196.6976 116.0272) (end 197.0024 115.7224) (width 0.254) (layer F.Cu) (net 10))
 (segment (start 196.6976 116.4336) (end 196.6976 116.0272) (width 0.254) (layer F.Cu) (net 10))
 (segment (start 197.1548 116.8908) (end 196.6976 116.4336) (width 0.254) (layer F.Cu) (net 10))
 (segment (start 198.7296 116.8908) (end 197.1548 116.8908) (width 0.254) (layer F.Cu) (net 10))
 (segment (start 199.1868 117.348) (end 198.7296 116.8908) (width 0.254) (layer F.Cu) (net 10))
 (segment (start 199.1868 117.9576) (end 199.1868 117.348) (width 0.254) (layer F.Cu) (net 10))
 (segment (start 198.8312 118.3132) (end 199.1868 117.9576) (width 0.254) (layer F.Cu) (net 10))
 (segment (start 198.1708 118.3132) (end 198.8312 118.3132) (width 0.254) (layer F.Cu) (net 10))
 (segment (start 197.303296 119.180704) (end 198.1708 118.3132) (width 0.254) (layer F.Cu) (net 10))
 (segment (start 196.088 115.1509) (end 197.1548 115.1509) (width 0.254) (layer F.Cu) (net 10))
 (segment (start 197.1548 115.1509) (end 197.4723 115.1509) (width 0.254) (layer F.Cu) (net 10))
 (segment (start 197.4723 115.1509) (end 198.628 115.1509) (width 0.254) (layer F.Cu) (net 10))
 (segment (start 197.303296 121.539256) (end 197.332344 121.539256) (width 0.254) (layer B.Cu) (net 10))
 (segment (start 197.332344 121.539256) (end 200.152 118.7196) (width 0.254) (layer B.Cu) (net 10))
 (segment (start 200.152 118.7196) (end 200.152 112.2172) (width 0.254) (layer B.Cu) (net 10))
 (segment (start 200.152 112.2172) (end 200.7108 111.6584) (width 0.254) (layer B.Cu) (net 10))
 (segment (start 200.7108 111.6584) (end 200.7108 108.6993) (width 0.254) (layer B.Cu) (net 10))
 (segment (start 200.7108 108.6993) (end 200.1012 108.0897) (width 0.254) (layer B.Cu) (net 10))
 (segment (start 197.9168 108.0897) (end 200.1012 108.0897) (width 0.254) (layer B.Cu) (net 10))
 (segment (start 195.58 108.0897) (end 197.9168 108.0897) (width 0.254) (layer B.Cu) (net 10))
 (segment (start 195.58 106.1847) (end 195.58 105.8164) (width 0.254) (layer B.Cu) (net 7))
 (segment (start 194.818 104.9528) (end 194.818 103.9368) (width 0.254) (layer F.Cu) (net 7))
 (segment (start 194.7672 105.0036) (end 194.818 104.9528) (width 0.254) (layer F.Cu) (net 7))
 (via (at 194.7672 105.0036) (size 0.889) (layers F.Cu B.Cu) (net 7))
 (segment (start 195.58 105.8164) (end 194.7672 105.0036) (width 0.254) (layer B.Cu) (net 7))
 (segment (start 197.9168 106.1847) (end 197.9168 105.5624) (width 0.254) (layer B.Cu) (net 9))
 (segment (start 197.358 105.0036) (end 197.358 103.9368) (width 0.254) (layer F.Cu) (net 9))
 (via (at 197.358 105.0036) (size 0.889) (layers F.Cu B.Cu) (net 9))
 (segment (start 197.9168 105.5624) (end 197.358 105.0036) (width 0.254) (layer B.Cu) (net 9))
 (segment (start 200.1012 106.1847) (end 200.1012 105.2068) (width 0.254) (layer B.Cu) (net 6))
 (segment (start 199.898 105.0036) (end 199.898 103.9368) (width 0.254) (layer F.Cu) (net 6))
 (via (at 199.898 105.0036) (size 0.889) (layers F.Cu B.Cu) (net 6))
 (segment (start 200.1012 105.2068) (end 199.898 105.0036) (width 0.254) (layer B.Cu) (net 6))
 (segment (start 198.628 110.2868) (end 198.628 110.5408) (width 0.254) (layer F.Cu) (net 4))
 (segment (start 197.5612 112.1791) (end 198.628 113.2459) (width 0.254) (layer F.Cu) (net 4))
 (segment (start 197.5612 111.6076) (end 197.5612 112.1791) (width 0.254) (layer F.Cu) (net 4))
 (segment (start 198.628 110.5408) (end 197.5612 111.6076) (width 0.254) (layer F.Cu) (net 4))
 (segment (start 196.088 110.2868) (end 196.088 113.2459) (width 0.254) (layer F.Cu) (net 3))
 (segment (start 193.548 106.1847) (end 192.0875 106.1847) (width 0.254) (layer B.Cu) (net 8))
 (via (at 192.0748 106.172) (size 0.889) (layers F.Cu B.Cu) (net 8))
 (segment (start 192.0875 106.1847) (end 192.0748 106.172) (width 0.254) (layer B.Cu) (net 8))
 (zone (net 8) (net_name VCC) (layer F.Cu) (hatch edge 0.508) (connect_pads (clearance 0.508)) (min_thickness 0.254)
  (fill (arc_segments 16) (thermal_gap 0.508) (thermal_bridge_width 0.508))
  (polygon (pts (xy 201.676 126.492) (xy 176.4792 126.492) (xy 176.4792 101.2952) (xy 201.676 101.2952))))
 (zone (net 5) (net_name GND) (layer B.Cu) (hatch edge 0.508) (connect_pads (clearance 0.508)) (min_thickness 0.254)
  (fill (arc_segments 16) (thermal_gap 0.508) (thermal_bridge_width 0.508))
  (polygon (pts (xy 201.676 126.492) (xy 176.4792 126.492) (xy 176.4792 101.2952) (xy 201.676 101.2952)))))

